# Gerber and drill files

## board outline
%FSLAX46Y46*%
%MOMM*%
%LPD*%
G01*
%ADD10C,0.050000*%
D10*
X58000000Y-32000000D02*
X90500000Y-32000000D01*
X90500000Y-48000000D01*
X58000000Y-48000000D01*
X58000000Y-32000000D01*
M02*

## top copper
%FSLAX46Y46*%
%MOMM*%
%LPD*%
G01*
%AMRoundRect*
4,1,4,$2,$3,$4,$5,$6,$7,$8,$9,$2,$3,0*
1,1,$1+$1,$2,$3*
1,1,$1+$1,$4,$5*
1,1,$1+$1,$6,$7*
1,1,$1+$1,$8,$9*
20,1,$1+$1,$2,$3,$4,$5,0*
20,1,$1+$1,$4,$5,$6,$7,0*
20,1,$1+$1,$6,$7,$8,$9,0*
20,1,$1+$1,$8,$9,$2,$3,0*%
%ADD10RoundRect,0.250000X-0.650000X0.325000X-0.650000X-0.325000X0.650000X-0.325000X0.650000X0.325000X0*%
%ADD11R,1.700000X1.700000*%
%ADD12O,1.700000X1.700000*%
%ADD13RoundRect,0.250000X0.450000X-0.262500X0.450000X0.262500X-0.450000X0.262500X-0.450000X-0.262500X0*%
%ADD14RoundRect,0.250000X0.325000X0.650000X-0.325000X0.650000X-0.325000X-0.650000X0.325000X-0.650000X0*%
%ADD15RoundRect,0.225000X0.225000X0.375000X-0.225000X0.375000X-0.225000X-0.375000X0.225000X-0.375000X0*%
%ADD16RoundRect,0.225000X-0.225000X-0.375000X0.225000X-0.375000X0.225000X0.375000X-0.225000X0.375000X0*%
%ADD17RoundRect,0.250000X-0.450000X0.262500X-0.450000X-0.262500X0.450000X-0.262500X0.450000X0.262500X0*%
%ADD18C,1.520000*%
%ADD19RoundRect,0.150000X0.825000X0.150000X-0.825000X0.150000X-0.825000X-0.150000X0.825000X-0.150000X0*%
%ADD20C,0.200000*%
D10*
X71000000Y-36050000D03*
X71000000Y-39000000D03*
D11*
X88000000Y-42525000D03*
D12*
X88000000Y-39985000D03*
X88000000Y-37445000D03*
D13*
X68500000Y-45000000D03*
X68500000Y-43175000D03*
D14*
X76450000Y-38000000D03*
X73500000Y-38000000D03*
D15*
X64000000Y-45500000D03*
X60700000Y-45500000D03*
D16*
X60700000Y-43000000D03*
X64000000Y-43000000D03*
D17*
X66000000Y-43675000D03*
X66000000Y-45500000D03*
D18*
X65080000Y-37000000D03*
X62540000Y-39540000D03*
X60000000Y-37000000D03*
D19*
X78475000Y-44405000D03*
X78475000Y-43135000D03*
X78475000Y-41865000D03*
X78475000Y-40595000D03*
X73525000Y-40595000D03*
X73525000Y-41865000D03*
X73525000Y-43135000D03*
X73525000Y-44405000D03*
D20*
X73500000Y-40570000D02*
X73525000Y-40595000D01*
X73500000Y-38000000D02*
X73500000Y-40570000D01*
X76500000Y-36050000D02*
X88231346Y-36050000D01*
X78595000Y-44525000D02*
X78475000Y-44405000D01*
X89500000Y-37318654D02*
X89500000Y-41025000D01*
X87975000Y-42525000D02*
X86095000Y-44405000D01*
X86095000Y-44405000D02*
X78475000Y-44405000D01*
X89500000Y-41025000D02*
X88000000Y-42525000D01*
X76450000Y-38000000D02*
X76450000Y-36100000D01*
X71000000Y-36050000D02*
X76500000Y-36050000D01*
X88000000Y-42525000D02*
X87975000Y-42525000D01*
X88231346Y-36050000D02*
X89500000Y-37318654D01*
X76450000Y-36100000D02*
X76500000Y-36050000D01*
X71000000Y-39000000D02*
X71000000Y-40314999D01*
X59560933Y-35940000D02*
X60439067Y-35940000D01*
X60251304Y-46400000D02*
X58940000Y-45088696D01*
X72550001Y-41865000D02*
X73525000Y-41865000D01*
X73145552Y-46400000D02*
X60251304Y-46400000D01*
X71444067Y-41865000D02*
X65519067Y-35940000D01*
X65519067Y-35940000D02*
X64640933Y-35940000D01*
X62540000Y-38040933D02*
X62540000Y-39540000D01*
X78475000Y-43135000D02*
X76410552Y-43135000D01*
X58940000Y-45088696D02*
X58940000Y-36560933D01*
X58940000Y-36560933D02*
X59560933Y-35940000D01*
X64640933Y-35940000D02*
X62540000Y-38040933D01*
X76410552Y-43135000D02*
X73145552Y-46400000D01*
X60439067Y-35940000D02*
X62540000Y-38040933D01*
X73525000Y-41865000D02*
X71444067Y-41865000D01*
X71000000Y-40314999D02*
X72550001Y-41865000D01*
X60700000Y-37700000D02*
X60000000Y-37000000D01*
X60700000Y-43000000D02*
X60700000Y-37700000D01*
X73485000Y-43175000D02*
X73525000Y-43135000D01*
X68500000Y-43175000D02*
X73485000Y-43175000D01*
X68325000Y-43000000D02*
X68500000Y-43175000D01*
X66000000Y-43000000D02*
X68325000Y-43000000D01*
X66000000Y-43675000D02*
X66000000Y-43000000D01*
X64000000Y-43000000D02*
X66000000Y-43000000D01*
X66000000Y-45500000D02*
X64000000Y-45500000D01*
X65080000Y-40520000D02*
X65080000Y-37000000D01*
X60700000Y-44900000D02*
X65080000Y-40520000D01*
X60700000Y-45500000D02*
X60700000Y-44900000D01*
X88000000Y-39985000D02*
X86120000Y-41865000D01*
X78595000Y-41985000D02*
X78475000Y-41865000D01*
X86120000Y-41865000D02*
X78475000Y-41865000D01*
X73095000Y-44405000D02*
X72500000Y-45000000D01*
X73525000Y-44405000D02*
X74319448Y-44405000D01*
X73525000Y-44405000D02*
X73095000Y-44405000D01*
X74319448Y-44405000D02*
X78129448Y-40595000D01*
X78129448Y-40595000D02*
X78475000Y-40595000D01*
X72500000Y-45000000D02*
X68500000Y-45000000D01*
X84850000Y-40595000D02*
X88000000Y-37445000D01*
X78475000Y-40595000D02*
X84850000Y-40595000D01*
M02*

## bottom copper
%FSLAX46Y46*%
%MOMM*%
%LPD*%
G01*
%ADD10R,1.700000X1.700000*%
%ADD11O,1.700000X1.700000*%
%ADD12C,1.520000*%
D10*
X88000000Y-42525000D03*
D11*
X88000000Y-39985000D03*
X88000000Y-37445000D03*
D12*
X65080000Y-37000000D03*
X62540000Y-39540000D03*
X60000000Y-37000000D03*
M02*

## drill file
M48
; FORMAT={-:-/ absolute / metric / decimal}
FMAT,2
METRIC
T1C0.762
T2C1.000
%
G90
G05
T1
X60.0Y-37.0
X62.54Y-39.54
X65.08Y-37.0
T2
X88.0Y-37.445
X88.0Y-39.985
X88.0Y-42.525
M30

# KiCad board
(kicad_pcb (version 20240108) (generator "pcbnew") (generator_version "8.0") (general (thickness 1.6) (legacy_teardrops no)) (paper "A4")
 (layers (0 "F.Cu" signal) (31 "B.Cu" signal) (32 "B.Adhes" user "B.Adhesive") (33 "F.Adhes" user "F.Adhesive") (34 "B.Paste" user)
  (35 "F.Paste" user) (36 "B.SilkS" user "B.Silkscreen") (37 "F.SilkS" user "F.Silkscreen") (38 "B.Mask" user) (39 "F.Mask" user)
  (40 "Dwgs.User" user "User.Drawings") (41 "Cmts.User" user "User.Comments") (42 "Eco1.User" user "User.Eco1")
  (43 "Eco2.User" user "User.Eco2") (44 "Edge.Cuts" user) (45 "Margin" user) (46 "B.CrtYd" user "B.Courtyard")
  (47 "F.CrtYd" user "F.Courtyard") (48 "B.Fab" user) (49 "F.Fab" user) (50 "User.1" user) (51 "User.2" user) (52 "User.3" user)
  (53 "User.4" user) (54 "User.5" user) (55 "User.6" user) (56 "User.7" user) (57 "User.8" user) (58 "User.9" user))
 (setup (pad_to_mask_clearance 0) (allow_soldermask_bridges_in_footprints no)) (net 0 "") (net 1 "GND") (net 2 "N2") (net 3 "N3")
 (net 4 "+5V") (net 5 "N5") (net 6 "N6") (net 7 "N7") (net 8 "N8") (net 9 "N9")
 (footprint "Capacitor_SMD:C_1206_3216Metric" (layer "F.Cu") (at 71 37.525 -90)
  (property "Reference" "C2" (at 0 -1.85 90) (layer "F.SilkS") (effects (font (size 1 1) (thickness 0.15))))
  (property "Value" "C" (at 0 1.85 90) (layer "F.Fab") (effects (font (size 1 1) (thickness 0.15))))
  (pad "1" smd roundrect (at -1.475 0 270) (size 1.15 1.8) (layers "F.Cu" "F.Paste" "F.Mask") (roundrect_rratio 0.217391) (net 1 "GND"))
  (pad "2" smd roundrect (at 1.475 0 270) (size 1.15 1.8) (layers "F.Cu" "F.Paste" "F.Mask") (roundrect_rratio 0.217391) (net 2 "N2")))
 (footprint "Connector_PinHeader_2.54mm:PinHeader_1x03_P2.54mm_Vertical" (layer "F.Cu") (at 88 42.525 180)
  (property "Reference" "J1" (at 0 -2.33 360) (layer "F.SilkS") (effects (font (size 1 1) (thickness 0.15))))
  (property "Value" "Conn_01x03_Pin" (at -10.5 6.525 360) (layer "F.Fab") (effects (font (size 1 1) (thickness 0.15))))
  (pad "1" thru_hole rect (at 0 0 180) (size 1.7 1.7) (drill 1) (layers "*.Cu" "*.Mask") (remove_unused_layers no) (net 1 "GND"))
  (pad "2" thru_hole oval (at 0 2.54 180) (size 1.7 1.7) (drill 1) (layers "*.Cu" "*.Mask") (remove_unused_layers no) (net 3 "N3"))
  (pad "3" thru_hole oval (at 0 5.08 180) (size 1.7 1.7) (drill 1) (layers "*.Cu" "*.Mask") (remove_unused_layers no) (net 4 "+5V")))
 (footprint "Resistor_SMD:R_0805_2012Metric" (layer "F.Cu") (at 68.5 44.0875 90)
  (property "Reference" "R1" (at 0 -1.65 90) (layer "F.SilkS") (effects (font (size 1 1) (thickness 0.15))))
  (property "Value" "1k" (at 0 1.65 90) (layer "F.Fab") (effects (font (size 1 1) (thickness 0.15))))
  (pad "1" smd roundrect (at -0.9125 0 90) (size 1.025 1.4) (layers "F.Cu" "F.Paste" "F.Mask") (roundrect_rratio 0.243902) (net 4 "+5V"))
  (pad "2" smd roundrect (at 0.9125 0 90) (size 1.025 1.4) (layers "F.Cu" "F.Paste" "F.Mask") (roundrect_rratio 0.243902) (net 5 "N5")))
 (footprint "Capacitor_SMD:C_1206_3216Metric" (layer "F.Cu") (at 74.975 38 180)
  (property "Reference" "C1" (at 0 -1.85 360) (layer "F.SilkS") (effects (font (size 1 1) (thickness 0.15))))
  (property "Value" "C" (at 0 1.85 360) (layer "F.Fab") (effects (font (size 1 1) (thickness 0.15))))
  (pad "1" smd roundrect (at -1.475 0 180) (size 1.15 1.8) (layers "F.Cu" "F.Paste" "F.Mask") (roundrect_rratio 0.217391) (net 1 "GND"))
  (pad "2" smd roundrect (at 1.475 0 180) (size 1.15 1.8) (layers "F.Cu" "F.Paste" "F.Mask") (roundrect_rratio 0.217391) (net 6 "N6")))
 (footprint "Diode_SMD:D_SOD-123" (layer "F.Cu") (at 62.35 45.5 180)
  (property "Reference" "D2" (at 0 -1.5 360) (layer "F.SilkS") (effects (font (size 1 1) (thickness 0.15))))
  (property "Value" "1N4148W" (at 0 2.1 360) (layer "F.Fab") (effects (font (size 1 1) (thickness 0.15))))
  (pad "1" smd roundrect (at -1.65 0 180) (size 0.9 1.2) (layers "F.Cu" "F.Paste" "F.Mask") (roundrect_rratio 0.25) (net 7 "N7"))
  (pad "2" smd roundrect (at 1.65 0 180) (size 0.9 1.2) (layers "F.Cu" "F.Paste" "F.Mask") (roundrect_rratio 0.25) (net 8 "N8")))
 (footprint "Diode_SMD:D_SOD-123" (layer "F.Cu") (at 62.35 43)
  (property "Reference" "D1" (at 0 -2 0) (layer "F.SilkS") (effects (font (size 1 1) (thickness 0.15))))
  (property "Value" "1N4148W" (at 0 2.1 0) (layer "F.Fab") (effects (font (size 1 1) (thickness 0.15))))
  (pad "1" smd roundrect (at -1.65 0) (size 0.9 1.2) (layers "F.Cu" "F.Paste" "F.Mask") (roundrect_rratio 0.25) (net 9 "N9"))
  (pad "2" smd roundrect (at 1.65 0) (size 0.9 1.2) (layers "F.Cu" "F.Paste" "F.Mask") (roundrect_rratio 0.25) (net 5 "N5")))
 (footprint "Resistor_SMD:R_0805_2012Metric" (layer "F.Cu") (at 66 44.5875 -90)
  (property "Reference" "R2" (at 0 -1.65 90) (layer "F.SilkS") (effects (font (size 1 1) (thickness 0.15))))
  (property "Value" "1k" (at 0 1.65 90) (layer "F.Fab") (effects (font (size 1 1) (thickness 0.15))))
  (pad "1" smd roundrect (at -0.9125 0 270) (size 1.025 1.4) (layers "F.Cu" "F.Paste" "F.Mask") (roundrect_rratio 0.243902) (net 5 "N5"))
  (pad "2" smd roundrect (at 0.9125 0 270) (size 1.025 1.4) (layers "F.Cu" "F.Paste" "F.Mask") (roundrect_rratio 0.243902) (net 7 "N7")))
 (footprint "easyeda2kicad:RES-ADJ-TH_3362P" (layer "F.Cu") (at 62.54 38.27 180)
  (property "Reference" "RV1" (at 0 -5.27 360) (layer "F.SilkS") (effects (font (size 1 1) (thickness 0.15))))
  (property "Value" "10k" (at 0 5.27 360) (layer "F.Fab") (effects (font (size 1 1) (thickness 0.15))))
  (pad "1" thru_hole circle (at -2.54 1.27 180) (size 1.52 1.52) (drill 0.762) (layers "*.Cu" "*.Mask") (remove_unused_layers no)
   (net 8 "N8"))
  (pad "2" thru_hole circle (at 0 -1.27 180) (size 1.52 1.52) (drill 0.762) (layers "*.Cu" "*.Mask") (remove_unused_layers no) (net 2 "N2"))
  (pad "3" thru_hole circle (at 2.54 1.27 180) (size 1.52 1.52) (drill 0.762) (layers "*.Cu" "*.Mask") (remove_unused_layers no)
   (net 9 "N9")))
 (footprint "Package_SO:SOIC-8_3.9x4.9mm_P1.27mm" (layer "F.Cu") (at 76 42.5 180)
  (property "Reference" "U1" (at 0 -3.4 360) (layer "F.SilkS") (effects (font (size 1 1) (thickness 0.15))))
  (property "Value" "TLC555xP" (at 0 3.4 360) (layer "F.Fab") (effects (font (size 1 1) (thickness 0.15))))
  (pad "1" smd roundrect (at -2.475 -1.905 180) (size 1.95 0.6) (layers "F.Cu" "F.Paste" "F.Mask") (roundrect_rratio 0.25) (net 1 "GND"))
  (pad "2" smd roundrect (at -2.475 -0.635 180) (size 1.95 0.6) (layers "F.Cu" "F.Paste" "F.Mask") (roundrect_rratio 0.25) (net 2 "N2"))
  (pad "3" smd roundrect (at -2.475 0.635 180) (size 1.95 0.6) (layers "F.Cu" "F.Paste" "F.Mask") (roundrect_rratio 0.25) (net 3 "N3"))
  (pad "4" smd roundrect (at -2.475 1.905 180) (size 1.95 0.6) (layers "F.Cu" "F.Paste" "F.Mask") (roundrect_rratio 0.25) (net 4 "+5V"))
  (pad "5" smd roundrect (at 2.475 1.905 180) (size 1.95 0.6) (layers "F.Cu" "F.Paste" "F.Mask") (roundrect_rratio 0.25) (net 6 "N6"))
  (pad "6" smd roundrect (at 2.475 0.635 180) (size 1.95 0.6) (layers "F.Cu" "F.Paste" "F.Mask") (roundrect_rratio 0.25) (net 2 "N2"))
  (pad "7" smd roundrect (at 2.475 -0.635 180) (size 1.95 0.6) (layers "F.Cu" "F.Paste" "F.Mask") (roundrect_rratio 0.25) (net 5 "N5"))
  (pad "8" smd roundrect (at 2.475 -1.905 180) (size 1.95 0.6) (layers "F.Cu" "F.Paste" "F.Mask") (roundrect_rratio 0.25) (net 4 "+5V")))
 (gr_rect (start 58 32) (end 90.5 48) (stroke (width 0.05) (type default)) (fill none) (layer "Edge.Cuts"))
 (segment (start 73.5 40.57) (end 73.525 40.595) (width 0.2) (layer "F.Cu") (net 6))
 (segment (start 73.5 38) (end 73.5 40.57) (width 0.2) (layer "F.Cu") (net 6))
 (segment (start 76.5 36.05) (end 88.231346 36.05) (width 0.2) (layer "F.Cu") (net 1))
 (segment (start 78.595 44.525) (end 78.475 44.405) (width 0.2) (layer "F.Cu") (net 1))
 (segment (start 89.5 37.318654) (end 89.5 41.025) (width 0.2) (layer "F.Cu") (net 1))
 (segment (start 87.975 42.525) (end 86.095 44.405) (width 0.2) (layer "F.Cu") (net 1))
 (segment (start 86.095 44.405) (end 78.475 44.405) (width 0.2) (layer "F.Cu") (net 1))
 (segment (start 89.5 41.025) (end 88 42.525) (width 0.2) (layer "F.Cu") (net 1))
 (segment (start 76.45 38) (end 76.45 36.1) (width 0.2) (layer "F.Cu") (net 1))
 (segment (start 71 36.05) (end 76.5 36.05) (width 0.2) (layer "F.Cu") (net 1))
 (segment (start 88 42.525) (end 87.975 42.525) (width 0.2) (layer "F.Cu") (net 1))
 (segment (start 88.231346 36.05) (end 89.5 37.318654) (width 0.2) (layer "F.Cu") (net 1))
 (segment (start 76.45 36.1) (end 76.5 36.05) (width 0.2) (layer "F.Cu") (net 1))
 (segment (start 71 39) (end 71 40.314999) (width 0.2) (layer "F.Cu") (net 2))
 (segment (start 59.560933 35.94) (end 60.439067 35.94) (width 0.2) (layer "F.Cu") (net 2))
 (segment (start 60.251304 46.4) (end 58.94 45.088696) (width 0.2) (layer "F.Cu") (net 2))
 (segment (start 72.550001 41.865) (end 73.525 41.865) (width 0.2) (layer "F.Cu") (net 2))
 (segment (start 73.145552 46.4) (end 60.251304 46.4) (width 0.2) (layer "F.Cu") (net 2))
 (segment (start 71.444067 41.865) (end 65.519067 35.94) (width 0.2) (layer "F.Cu") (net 2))
 (segment (start 65.519067 35.94) (end 64.640933 35.94) (width 0.2) (layer "F.Cu") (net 2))
 (segment (start 62.54 38.040933) (end 62.54 39.54) (width 0.2) (layer "F.Cu") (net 2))
 (segment (start 78.475 43.135) (end 76.410552 43.135) (width 0.2) (layer "F.Cu") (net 2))
 (segment (start 58.94 45.088696) (end 58.94 36.560933) (width 0.2) (layer "F.Cu") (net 2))
 (segment (start 58.94 36.560933) (end 59.560933 35.94) (width 0.2) (layer "F.Cu") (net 2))
 (segment (start 64.640933 35.94) (end 62.54 38.040933) (width 0.2) (layer "F.Cu") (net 2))
 (segment (start 76.410552 43.135) (end 73.145552 46.4) (width 0.2) (layer "F.Cu") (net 2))
 (segment (start 60.439067 35.94) (end 62.54 38.040933) (width 0.2) (layer "F.Cu") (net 2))
 (segment (start 73.525 41.865) (end 71.444067 41.865) (width 0.2) (layer "F.Cu") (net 2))
 (segment (start 71 40.314999) (end 72.550001 41.865) (width 0.2) (layer "F.Cu") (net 2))
 (segment (start 60.7 37.7) (end 60 37) (width 0.2) (layer "F.Cu") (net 9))
 (segment (start 60.7 43) (end 60.7 37.7) (width 0.2) (layer "F.Cu") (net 9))
 (segment (start 73.485 43.175) (end 73.525 43.135) (width 0.2) (layer "F.Cu") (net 5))
 (segment (start 68.5 43.175) (end 73.485 43.175) (width 0.2) (layer "F.Cu") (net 5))
 (segment (start 68.325 43) (end 68.5 43.175) (width 0.2) (layer "F.Cu") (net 5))
 (segment (start 66 43) (end 68.325 43) (width 0.2) (layer "F.Cu") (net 5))
 (segment (start 66 43.675) (end 66 43) (width 0.2) (layer "F.Cu") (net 5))
 (segment (start 64 43) (end 66 43) (width 0.2) (layer "F.Cu") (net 5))
 (segment (start 66 45.5) (end 64 45.5) (width 0.2) (layer "F.Cu") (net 7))
 (segment (start 65.08 40.52) (end 65.08 37) (width 0.2) (layer "F.Cu") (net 8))
 (segment (start 60.7 44.9) (end 65.08 40.52) (width 0.2) (layer "F.Cu") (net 8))
 (segment (start 60.7 45.5) (end 60.7 44.9) (width 0.2) (layer "F.Cu") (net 8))
 (segment (start 88 39.985) (end 86.12 41.865) (width 0.2) (layer "F.Cu") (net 3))
 (segment (start 78.595 41.985) (end 78.475 41.865) (width 0.2) (layer "F.Cu") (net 3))
 (segment (start 86.12 41.865) (end 78.475 41.865) (width 0.2) (layer "F.Cu") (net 3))
 (segment (start 73.095 44.405) (end 72.5 45) (width 0.2) (layer "F.Cu") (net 4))
 (segment (start 73.525 44.405) (end 74.319448 44.405) (width 0.2) (layer "F.Cu") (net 4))
 (segment (start 73.525 44.405) (end 73.095 44.405) (width 0.2) (layer "F.Cu") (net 4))
 (segment (start 74.319448 44.405) (end 78.129448 40.595) (width 0.2) (layer "F.Cu") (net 4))
 (segment (start 78.129448 40.595) (end 78.475 40.595) (width 0.2) (layer "F.Cu") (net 4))
 (segment (start 72.5 45) (end 68.5 45) (width 0.2) (layer "F.Cu") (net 4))
 (segment (start 84.85 40.595) (end 88 37.445) (width 0.2) (layer "F.Cu") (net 4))
 (segment (start 78.475 40.595) (end 84.85 40.595) (width 0.2) (layer "F.Cu") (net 4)))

